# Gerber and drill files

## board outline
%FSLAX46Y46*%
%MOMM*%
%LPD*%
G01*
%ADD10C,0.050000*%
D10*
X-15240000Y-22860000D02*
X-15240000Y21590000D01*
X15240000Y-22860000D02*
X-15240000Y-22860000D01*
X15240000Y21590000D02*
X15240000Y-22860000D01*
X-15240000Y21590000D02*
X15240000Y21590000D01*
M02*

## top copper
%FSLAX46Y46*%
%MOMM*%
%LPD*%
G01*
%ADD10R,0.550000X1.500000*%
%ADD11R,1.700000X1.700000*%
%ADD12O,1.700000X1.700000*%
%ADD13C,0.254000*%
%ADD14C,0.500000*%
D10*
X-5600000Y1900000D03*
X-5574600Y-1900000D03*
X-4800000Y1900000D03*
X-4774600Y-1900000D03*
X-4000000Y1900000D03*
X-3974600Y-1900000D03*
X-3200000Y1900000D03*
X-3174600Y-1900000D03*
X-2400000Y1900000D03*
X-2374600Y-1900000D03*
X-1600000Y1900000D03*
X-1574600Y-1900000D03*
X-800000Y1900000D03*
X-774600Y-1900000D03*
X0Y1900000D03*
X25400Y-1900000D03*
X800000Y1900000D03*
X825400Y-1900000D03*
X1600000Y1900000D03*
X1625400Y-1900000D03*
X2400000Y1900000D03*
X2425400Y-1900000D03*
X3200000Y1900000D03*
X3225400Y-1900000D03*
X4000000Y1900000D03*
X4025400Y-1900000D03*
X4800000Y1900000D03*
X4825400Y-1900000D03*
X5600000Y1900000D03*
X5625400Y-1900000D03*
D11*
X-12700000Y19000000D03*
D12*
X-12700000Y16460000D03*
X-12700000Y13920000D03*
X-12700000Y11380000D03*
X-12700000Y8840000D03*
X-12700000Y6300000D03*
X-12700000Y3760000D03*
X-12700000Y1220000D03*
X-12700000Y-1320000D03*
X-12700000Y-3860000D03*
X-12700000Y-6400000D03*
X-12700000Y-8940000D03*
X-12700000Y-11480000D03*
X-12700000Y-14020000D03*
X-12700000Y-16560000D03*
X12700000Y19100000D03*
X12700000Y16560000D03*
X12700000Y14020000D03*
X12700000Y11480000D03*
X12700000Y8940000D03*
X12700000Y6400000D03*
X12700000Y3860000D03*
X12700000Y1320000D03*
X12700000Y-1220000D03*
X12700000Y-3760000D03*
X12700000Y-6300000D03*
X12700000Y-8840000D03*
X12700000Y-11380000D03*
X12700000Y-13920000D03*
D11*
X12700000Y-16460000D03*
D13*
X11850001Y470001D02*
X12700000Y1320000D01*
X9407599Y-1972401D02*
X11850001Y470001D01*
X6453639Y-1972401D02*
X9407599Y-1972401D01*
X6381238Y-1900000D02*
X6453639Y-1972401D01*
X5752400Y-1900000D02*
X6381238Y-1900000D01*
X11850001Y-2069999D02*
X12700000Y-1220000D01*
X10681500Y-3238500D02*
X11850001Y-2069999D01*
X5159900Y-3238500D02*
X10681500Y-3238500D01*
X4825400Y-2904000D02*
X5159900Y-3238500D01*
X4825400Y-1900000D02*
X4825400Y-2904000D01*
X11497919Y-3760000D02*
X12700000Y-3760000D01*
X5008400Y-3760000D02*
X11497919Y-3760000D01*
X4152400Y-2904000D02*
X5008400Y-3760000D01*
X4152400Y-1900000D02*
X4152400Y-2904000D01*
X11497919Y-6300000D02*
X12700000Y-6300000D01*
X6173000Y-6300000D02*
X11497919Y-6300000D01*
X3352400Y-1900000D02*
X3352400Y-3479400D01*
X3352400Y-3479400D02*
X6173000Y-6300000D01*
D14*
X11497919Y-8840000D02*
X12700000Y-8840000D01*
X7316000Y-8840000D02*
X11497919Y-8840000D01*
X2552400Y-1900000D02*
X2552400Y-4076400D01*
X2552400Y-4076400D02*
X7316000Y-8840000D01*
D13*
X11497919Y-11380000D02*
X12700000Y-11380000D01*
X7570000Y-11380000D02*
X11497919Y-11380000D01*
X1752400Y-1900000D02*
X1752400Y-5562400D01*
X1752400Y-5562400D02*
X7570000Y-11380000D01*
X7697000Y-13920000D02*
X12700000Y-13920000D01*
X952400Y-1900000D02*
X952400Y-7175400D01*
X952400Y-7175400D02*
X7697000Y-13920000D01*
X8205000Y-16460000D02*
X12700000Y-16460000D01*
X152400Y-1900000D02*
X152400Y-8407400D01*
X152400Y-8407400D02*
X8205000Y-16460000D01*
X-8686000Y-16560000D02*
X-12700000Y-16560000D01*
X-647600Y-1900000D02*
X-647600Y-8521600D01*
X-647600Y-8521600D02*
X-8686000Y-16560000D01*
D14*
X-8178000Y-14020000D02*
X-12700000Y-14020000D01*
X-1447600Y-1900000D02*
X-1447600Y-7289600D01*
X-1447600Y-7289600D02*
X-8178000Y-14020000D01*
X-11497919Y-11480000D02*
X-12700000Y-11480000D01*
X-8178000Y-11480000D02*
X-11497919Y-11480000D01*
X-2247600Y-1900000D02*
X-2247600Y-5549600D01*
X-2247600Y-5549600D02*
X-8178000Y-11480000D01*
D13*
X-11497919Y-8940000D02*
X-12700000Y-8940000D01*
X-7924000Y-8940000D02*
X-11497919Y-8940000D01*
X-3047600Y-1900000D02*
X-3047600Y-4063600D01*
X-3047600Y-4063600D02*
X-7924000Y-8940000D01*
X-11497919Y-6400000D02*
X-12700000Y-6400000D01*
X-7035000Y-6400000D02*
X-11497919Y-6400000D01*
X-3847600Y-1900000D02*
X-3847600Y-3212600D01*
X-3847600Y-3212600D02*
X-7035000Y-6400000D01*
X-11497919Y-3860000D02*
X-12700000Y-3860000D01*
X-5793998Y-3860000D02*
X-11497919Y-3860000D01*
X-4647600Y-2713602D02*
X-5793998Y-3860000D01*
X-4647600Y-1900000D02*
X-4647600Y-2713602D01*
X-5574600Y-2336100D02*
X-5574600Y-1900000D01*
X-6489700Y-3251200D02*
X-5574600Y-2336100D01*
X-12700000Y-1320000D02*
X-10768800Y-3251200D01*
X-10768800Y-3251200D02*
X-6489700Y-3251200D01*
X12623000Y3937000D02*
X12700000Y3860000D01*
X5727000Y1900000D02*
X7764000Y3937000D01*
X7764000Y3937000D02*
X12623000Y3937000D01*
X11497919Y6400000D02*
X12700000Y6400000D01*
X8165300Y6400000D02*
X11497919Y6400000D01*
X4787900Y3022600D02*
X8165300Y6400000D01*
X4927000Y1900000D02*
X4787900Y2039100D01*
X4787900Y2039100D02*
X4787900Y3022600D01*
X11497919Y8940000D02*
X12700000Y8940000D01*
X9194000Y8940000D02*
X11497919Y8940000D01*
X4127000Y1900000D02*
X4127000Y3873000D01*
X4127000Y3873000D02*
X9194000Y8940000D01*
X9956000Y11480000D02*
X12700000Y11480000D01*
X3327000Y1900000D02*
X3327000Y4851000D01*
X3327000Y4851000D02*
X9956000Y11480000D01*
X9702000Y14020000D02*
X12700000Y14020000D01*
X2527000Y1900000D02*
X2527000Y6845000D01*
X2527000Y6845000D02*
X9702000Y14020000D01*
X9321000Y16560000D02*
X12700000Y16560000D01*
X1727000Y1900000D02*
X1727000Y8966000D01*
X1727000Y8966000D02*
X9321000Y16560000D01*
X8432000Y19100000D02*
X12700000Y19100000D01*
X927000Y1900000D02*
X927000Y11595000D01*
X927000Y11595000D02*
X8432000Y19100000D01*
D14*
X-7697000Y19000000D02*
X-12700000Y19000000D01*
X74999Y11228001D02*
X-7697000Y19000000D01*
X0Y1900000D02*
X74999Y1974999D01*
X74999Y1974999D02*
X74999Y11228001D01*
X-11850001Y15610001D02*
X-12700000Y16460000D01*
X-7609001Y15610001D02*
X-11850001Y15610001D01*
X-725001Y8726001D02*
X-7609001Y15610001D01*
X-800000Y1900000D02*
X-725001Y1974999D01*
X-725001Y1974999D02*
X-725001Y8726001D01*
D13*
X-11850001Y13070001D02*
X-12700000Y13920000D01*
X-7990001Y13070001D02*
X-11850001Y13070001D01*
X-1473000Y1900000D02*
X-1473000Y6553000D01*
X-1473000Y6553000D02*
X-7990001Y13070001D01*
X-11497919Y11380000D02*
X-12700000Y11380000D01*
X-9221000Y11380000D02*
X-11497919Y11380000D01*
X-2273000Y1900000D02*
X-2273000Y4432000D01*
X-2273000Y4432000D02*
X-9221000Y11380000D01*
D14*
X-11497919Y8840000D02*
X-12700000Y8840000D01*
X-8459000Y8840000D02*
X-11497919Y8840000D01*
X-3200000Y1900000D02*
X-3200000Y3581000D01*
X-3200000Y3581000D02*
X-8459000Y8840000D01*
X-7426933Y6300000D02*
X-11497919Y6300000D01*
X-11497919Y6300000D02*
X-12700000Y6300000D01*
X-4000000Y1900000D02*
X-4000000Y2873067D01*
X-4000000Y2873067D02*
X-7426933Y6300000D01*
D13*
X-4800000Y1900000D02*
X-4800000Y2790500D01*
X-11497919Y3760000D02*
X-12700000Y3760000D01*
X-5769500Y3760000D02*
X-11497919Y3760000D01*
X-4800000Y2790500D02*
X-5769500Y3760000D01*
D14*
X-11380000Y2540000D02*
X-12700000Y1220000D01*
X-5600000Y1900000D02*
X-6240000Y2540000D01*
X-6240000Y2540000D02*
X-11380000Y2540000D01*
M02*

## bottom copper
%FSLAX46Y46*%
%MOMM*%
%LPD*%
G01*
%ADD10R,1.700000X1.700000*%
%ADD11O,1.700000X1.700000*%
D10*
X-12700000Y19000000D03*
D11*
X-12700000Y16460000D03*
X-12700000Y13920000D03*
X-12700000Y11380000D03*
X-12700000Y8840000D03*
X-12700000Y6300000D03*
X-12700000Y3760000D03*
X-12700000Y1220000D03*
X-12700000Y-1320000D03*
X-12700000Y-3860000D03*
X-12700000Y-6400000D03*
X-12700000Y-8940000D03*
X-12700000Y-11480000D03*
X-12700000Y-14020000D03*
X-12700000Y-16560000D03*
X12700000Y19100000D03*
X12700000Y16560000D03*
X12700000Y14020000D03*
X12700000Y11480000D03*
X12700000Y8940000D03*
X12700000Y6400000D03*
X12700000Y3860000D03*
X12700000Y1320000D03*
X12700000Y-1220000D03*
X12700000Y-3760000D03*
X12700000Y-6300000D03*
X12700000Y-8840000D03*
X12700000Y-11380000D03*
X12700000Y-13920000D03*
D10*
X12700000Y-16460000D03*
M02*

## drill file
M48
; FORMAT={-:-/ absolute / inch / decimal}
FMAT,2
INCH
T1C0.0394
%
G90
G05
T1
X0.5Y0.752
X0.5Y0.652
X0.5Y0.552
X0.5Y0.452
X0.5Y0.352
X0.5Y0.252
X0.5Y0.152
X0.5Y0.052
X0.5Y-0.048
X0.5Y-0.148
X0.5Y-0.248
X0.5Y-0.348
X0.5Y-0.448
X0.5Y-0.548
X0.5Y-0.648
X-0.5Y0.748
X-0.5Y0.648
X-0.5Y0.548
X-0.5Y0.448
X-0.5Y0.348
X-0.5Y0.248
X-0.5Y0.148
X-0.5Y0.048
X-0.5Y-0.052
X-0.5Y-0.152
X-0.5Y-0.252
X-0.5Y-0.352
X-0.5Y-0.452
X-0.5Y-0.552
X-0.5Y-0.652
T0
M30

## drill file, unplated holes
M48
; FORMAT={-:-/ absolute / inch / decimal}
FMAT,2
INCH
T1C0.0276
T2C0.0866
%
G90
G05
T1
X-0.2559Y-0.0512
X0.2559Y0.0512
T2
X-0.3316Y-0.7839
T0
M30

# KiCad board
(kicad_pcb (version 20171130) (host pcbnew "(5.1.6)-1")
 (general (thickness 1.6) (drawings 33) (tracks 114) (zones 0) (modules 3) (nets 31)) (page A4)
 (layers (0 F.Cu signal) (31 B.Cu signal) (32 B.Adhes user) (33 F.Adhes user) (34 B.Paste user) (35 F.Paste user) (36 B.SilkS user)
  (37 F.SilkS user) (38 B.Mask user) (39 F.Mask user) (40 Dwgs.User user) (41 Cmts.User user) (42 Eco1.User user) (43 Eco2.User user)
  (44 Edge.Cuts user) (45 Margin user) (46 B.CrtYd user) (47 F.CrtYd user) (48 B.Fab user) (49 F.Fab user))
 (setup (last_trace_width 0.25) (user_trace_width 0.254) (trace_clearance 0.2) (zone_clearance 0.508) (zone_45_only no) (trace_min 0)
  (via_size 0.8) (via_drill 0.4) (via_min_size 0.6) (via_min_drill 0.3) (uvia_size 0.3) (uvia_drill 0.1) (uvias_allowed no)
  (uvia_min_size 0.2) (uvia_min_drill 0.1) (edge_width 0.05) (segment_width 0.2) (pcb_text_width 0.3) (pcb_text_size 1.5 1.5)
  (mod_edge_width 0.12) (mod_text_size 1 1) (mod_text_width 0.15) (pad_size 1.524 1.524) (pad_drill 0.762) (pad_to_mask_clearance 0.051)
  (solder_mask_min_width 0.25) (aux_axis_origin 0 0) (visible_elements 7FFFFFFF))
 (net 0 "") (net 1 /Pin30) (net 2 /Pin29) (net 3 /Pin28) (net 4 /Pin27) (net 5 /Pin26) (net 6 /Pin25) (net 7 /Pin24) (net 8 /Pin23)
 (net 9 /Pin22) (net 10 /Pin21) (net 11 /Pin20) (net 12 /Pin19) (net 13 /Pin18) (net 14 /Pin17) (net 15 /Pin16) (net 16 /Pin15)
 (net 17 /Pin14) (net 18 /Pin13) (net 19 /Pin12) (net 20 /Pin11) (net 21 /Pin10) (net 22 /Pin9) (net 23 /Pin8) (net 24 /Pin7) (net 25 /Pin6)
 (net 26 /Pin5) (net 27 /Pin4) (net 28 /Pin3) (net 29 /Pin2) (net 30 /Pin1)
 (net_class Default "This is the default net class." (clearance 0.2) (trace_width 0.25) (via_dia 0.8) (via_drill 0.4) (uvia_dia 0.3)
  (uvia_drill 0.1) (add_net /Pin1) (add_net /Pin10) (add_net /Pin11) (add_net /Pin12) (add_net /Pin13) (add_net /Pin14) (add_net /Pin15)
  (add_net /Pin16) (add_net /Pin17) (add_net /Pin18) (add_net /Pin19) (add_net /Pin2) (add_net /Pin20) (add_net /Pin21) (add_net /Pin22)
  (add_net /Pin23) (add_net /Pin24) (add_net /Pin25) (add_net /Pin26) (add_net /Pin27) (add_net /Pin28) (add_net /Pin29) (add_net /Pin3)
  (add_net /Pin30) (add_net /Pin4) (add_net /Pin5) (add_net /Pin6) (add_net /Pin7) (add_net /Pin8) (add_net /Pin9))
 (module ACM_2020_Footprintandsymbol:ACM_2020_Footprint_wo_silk (layer F.Cu) (at 0 0)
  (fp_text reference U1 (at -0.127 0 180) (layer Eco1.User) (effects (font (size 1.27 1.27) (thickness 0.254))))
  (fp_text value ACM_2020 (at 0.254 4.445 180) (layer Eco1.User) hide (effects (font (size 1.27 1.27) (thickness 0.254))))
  (pad 30 smd rect (at -5.6 -1.9) (size 0.55 1.5) (layers F.Cu F.Paste F.Mask) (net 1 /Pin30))
  (pad 29 smd rect (at -5.5746 1.9) (size 0.55 1.5) (layers F.Cu F.Paste F.Mask) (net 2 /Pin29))
  (pad 28 smd rect (at -4.8 -1.9) (size 0.55 1.5) (layers F.Cu F.Paste F.Mask) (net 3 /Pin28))
  (pad 27 smd rect (at -4.7746 1.9) (size 0.55 1.5) (layers F.Cu F.Paste F.Mask) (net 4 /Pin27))
  (pad 26 smd rect (at -4 -1.9) (size 0.55 1.5) (layers F.Cu F.Paste F.Mask) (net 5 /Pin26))
  (pad 25 smd rect (at -3.9746 1.9) (size 0.55 1.5) (layers F.Cu F.Paste F.Mask) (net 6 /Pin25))
  (pad 24 smd rect (at -3.2 -1.9) (size 0.55 1.5) (layers F.Cu F.Paste F.Mask) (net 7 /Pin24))
  (pad 23 smd rect (at -3.1746 1.9) (size 0.55 1.5) (layers F.Cu F.Paste F.Mask) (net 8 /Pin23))
  (pad 22 smd rect (at -2.4 -1.9) (size 0.55 1.5) (layers F.Cu F.Paste F.Mask) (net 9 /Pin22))
  (pad 21 smd rect (at -2.3746 1.9) (size 0.55 1.5) (layers F.Cu F.Paste F.Mask) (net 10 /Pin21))
  (pad 20 smd rect (at -1.6 -1.9) (size 0.55 1.5) (layers F.Cu F.Paste F.Mask) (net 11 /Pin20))
  (pad 19 smd rect (at -1.5746 1.9) (size 0.55 1.5) (layers F.Cu F.Paste F.Mask) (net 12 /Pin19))
  (pad 18 smd rect (at -0.8 -1.9) (size 0.55 1.5) (layers F.Cu F.Paste F.Mask) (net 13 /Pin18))
  (pad 17 smd rect (at -0.7746 1.9) (size 0.55 1.5) (layers F.Cu F.Paste F.Mask) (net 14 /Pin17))
  (pad 16 smd rect (at 0 -1.9) (size 0.55 1.5) (layers F.Cu F.Paste F.Mask) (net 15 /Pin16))
  (pad 15 smd rect (at 0.0254 1.9) (size 0.55 1.5) (layers F.Cu F.Paste F.Mask) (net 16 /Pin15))
  (pad 14 smd rect (at 0.8 -1.9) (size 0.55 1.5) (layers F.Cu F.Paste F.Mask) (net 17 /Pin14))
  (pad 13 smd rect (at 0.8254 1.9) (size 0.55 1.5) (layers F.Cu F.Paste F.Mask) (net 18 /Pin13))
  (pad 12 smd rect (at 1.6 -1.9) (size 0.55 1.5) (layers F.Cu F.Paste F.Mask) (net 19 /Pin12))
  (pad 11 smd rect (at 1.6254 1.9) (size 0.55 1.5) (layers F.Cu F.Paste F.Mask) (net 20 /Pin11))
  (pad 10 smd rect (at 2.4 -1.9) (size 0.55 1.5) (layers F.Cu F.Paste F.Mask) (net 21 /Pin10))
  (pad 9 smd rect (at 2.4254 1.9) (size 0.55 1.5) (layers F.Cu F.Paste F.Mask) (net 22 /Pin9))
  (pad 8 smd rect (at 3.2 -1.9) (size 0.55 1.5) (layers F.Cu F.Paste F.Mask) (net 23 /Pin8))
  (pad 7 smd rect (at 3.2254 1.9) (size 0.55 1.5) (layers F.Cu F.Paste F.Mask) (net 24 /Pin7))
  (pad 6 smd rect (at 4 -1.9) (size 0.55 1.5) (layers F.Cu F.Paste F.Mask) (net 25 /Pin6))
  (pad 5 smd rect (at 4.0254 1.9) (size 0.55 1.5) (layers F.Cu F.Paste F.Mask) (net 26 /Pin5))
  (pad 4 smd rect (at 4.8 -1.9) (size 0.55 1.5) (layers F.Cu F.Paste F.Mask) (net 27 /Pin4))
  (pad 3 smd rect (at 4.8254 1.9) (size 0.55 1.5) (layers F.Cu F.Paste F.Mask) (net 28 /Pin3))
  (pad 2 smd rect (at 5.6 -1.9) (size 0.55 1.5) (layers F.Cu F.Paste F.Mask) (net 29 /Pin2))
  (pad 1 smd rect (at 5.6254 1.9) (size 0.55 1.5) (layers F.Cu F.Paste F.Mask) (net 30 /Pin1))
  (pad "" np_thru_hole circle (at -6.5 1.3) (size 0.7 0.7) (drill 0.7) (layers *.Cu *.Mask))
  (pad "" np_thru_hole circle (at 6.5 -1.3) (size 0.7 0.7) (drill 0.7) (layers *.Cu *.Mask))
  (pad "" np_thru_hole circle (at -8.422 19.912) (size 2.2 2.2) (drill 2.2) (layers *.Cu *.Mask)))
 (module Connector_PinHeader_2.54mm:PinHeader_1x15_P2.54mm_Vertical (layer F.Cu) (at -12.7 -19)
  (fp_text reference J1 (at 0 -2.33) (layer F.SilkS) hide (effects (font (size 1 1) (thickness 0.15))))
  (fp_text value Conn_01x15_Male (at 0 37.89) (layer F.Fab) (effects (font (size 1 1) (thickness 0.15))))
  (pad 1 thru_hole rect (at 0 0) (size 1.7 1.7) (drill 1) (layers *.Cu *.Mask) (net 15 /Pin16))
  (pad 2 thru_hole oval (at 0 2.54) (size 1.7 1.7) (drill 1) (layers *.Cu *.Mask) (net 13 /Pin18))
  (pad 3 thru_hole oval (at 0 5.08) (size 1.7 1.7) (drill 1) (layers *.Cu *.Mask) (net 11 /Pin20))
  (pad 4 thru_hole oval (at 0 7.62) (size 1.7 1.7) (drill 1) (layers *.Cu *.Mask) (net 9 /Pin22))
  (pad 5 thru_hole oval (at 0 10.16) (size 1.7 1.7) (drill 1) (layers *.Cu *.Mask) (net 7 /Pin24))
  (pad 6 thru_hole oval (at 0 12.7) (size 1.7 1.7) (drill 1) (layers *.Cu *.Mask) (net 5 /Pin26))
  (pad 7 thru_hole oval (at 0 15.24) (size 1.7 1.7) (drill 1) (layers *.Cu *.Mask) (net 3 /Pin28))
  (pad 8 thru_hole oval (at 0 17.78) (size 1.7 1.7) (drill 1) (layers *.Cu *.Mask) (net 1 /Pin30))
  (pad 9 thru_hole oval (at 0 20.32) (size 1.7 1.7) (drill 1) (layers *.Cu *.Mask) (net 2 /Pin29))
  (pad 10 thru_hole oval (at 0 22.86) (size 1.7 1.7) (drill 1) (layers *.Cu *.Mask) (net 4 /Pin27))
  (pad 11 thru_hole oval (at 0 25.4) (size 1.7 1.7) (drill 1) (layers *.Cu *.Mask) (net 6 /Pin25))
  (pad 12 thru_hole oval (at 0 27.94) (size 1.7 1.7) (drill 1) (layers *.Cu *.Mask) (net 8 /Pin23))
  (pad 13 thru_hole oval (at 0 30.48) (size 1.7 1.7) (drill 1) (layers *.Cu *.Mask) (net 10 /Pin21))
  (pad 14 thru_hole oval (at 0 33.02) (size 1.7 1.7) (drill 1) (layers *.Cu *.Mask) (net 12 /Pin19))
  (pad 15 thru_hole oval (at 0 35.56) (size 1.7 1.7) (drill 1) (layers *.Cu *.Mask) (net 14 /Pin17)))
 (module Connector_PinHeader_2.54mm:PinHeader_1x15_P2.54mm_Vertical (layer F.Cu) (at 12.7 16.46 180)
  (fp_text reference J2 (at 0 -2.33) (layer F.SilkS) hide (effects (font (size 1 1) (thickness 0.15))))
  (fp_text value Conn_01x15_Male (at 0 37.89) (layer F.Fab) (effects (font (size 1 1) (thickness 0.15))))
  (pad 15 thru_hole oval (at 0 35.56 180) (size 1.7 1.7) (drill 1) (layers *.Cu *.Mask) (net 17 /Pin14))
  (pad 14 thru_hole oval (at 0 33.02 180) (size 1.7 1.7) (drill 1) (layers *.Cu *.Mask) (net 19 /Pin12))
  (pad 13 thru_hole oval (at 0 30.48 180) (size 1.7 1.7) (drill 1) (layers *.Cu *.Mask) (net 21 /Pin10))
  (pad 12 thru_hole oval (at 0 27.94 180) (size 1.7 1.7) (drill 1) (layers *.Cu *.Mask) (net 23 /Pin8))
  (pad 11 thru_hole oval (at 0 25.4 180) (size 1.7 1.7) (drill 1) (layers *.Cu *.Mask) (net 25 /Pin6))
  (pad 10 thru_hole oval (at 0 22.86 180) (size 1.7 1.7) (drill 1) (layers *.Cu *.Mask) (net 27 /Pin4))
  (pad 9 thru_hole oval (at 0 20.32 180) (size 1.7 1.7) (drill 1) (layers *.Cu *.Mask) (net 29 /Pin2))
  (pad 8 thru_hole oval (at 0 17.78 180) (size 1.7 1.7) (drill 1) (layers *.Cu *.Mask) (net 30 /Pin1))
  (pad 7 thru_hole oval (at 0 15.24 180) (size 1.7 1.7) (drill 1) (layers *.Cu *.Mask) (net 28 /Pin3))
  (pad 6 thru_hole oval (at 0 12.7 180) (size 1.7 1.7) (drill 1) (layers *.Cu *.Mask) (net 26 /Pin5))
  (pad 5 thru_hole oval (at 0 10.16 180) (size 1.7 1.7) (drill 1) (layers *.Cu *.Mask) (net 24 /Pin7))
  (pad 4 thru_hole oval (at 0 7.62 180) (size 1.7 1.7) (drill 1) (layers *.Cu *.Mask) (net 22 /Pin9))
  (pad 3 thru_hole oval (at 0 5.08 180) (size 1.7 1.7) (drill 1) (layers *.Cu *.Mask) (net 20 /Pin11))
  (pad 2 thru_hole oval (at 0 2.54 180) (size 1.7 1.7) (drill 1) (layers *.Cu *.Mask) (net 18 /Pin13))
  (pad 1 thru_hole rect (at 0 0 180) (size 1.7 1.7) (drill 1) (layers *.Cu *.Mask) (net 16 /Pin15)))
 (gr_line (start -15.24 22.86) (end -15.24 -21.59) (layer Edge.Cuts) (width 0.05))
 (gr_line (start 15.24 22.86) (end -15.24 22.86) (layer Edge.Cuts) (width 0.05))
 (gr_line (start 15.24 -21.59) (end 15.24 22.86) (layer Edge.Cuts) (width 0.05))
 (gr_line (start -15.24 -21.59) (end 15.24 -21.59) (layer Edge.Cuts) (width 0.05))
 (segment (start 11.850001 -0.470001) (end 12.7 -1.32) (width 0.254) (layer F.Cu) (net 30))
 (segment (start 9.407599 1.972401) (end 11.850001 -0.470001) (width 0.254) (layer F.Cu) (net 30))
 (segment (start 6.453639 1.972401) (end 9.407599 1.972401) (width 0.254) (layer F.Cu) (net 30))
 (segment (start 6.381238 1.9) (end 6.453639 1.972401) (width 0.254) (layer F.Cu) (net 30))
 (segment (start 5.7524 1.9) (end 6.381238 1.9) (width 0.254) (layer F.Cu) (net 30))
 (segment (start 11.850001 2.069999) (end 12.7 1.22) (width 0.254) (layer F.Cu) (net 28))
 (segment (start 10.6815 3.2385) (end 11.850001 2.069999) (width 0.254) (layer F.Cu) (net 28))
 (segment (start 5.1599 3.2385) (end 10.6815 3.2385) (width 0.254) (layer F.Cu) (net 28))
 (segment (start 4.8254 2.904) (end 5.1599 3.2385) (width 0.254) (layer F.Cu) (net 28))
 (segment (start 4.8254 1.9) (end 4.8254 2.904) (width 0.254) (layer F.Cu) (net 28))
 (segment (start 11.497919 3.76) (end 12.7 3.76) (width 0.254) (layer F.Cu) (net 26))
 (segment (start 5.0084 3.76) (end 11.497919 3.76) (width 0.254) (layer F.Cu) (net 26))
 (segment (start 4.1524 2.904) (end 5.0084 3.76) (width 0.254) (layer F.Cu) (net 26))
 (segment (start 4.1524 1.9) (end 4.1524 2.904) (width 0.254) (layer F.Cu) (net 26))
 (segment (start 11.497919 6.3) (end 12.7 6.3) (width 0.254) (layer F.Cu) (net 24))
 (segment (start 6.173 6.3) (end 11.497919 6.3) (width 0.254) (layer F.Cu) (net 24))
 (segment (start 3.3524 1.9) (end 3.3524 3.4794) (width 0.254) (layer F.Cu) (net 24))
 (segment (start 3.3524 3.4794) (end 6.173 6.3) (width 0.254) (layer F.Cu) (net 24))
 (segment (start 11.497919 8.84) (end 12.7 8.84) (width 0.5) (layer F.Cu) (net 22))
 (segment (start 7.316 8.84) (end 11.497919 8.84) (width 0.5) (layer F.Cu) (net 22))
 (segment (start 2.5524 1.9) (end 2.5524 4.0764) (width 0.5) (layer F.Cu) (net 22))
 (segment (start 2.5524 4.0764) (end 7.316 8.84) (width 0.5) (layer F.Cu) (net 22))
 (segment (start 11.497919 11.38) (end 12.7 11.38) (width 0.254) (layer F.Cu) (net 20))
 (segment (start 7.57 11.38) (end 11.497919 11.38) (width 0.254) (layer F.Cu) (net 20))
 (segment (start 1.7524 1.9) (end 1.7524 5.5624) (width 0.254) (layer F.Cu) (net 20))
 (segment (start 1.7524 5.5624) (end 7.57 11.38) (width 0.254) (layer F.Cu) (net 20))
 (segment (start 7.697 13.92) (end 12.7 13.92) (width 0.254) (layer F.Cu) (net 18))
 (segment (start 0.9524 1.9) (end 0.9524 7.1754) (width 0.254) (layer F.Cu) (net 18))
 (segment (start 0.9524 7.1754) (end 7.697 13.92) (width 0.254) (layer F.Cu) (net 18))
 (segment (start 8.205 16.46) (end 12.7 16.46) (width 0.254) (layer F.Cu) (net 16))
 (segment (start 0.1524 1.9) (end 0.1524 8.4074) (width 0.254) (layer F.Cu) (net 16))
 (segment (start 0.1524 8.4074) (end 8.205 16.46) (width 0.254) (layer F.Cu) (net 16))
 (segment (start -8.686 16.56) (end -12.7 16.56) (width 0.254) (layer F.Cu) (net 14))
 (segment (start -0.6476 1.9) (end -0.6476 8.5216) (width 0.254) (layer F.Cu) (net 14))
 (segment (start -0.6476 8.5216) (end -8.686 16.56) (width 0.254) (layer F.Cu) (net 14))
 (segment (start -8.178 14.02) (end -12.7 14.02) (width 0.5) (layer F.Cu) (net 12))
 (segment (start -1.4476 1.9) (end -1.4476 7.2896) (width 0.5) (layer F.Cu) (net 12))
 (segment (start -1.4476 7.2896) (end -8.178 14.02) (width 0.5) (layer F.Cu) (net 12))
 (segment (start -11.497919 11.48) (end -12.7 11.48) (width 0.5) (layer F.Cu) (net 10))
 (segment (start -8.178 11.48) (end -11.497919 11.48) (width 0.5) (layer F.Cu) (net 10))
 (segment (start -2.2476 1.9) (end -2.2476 5.5496) (width 0.5) (layer F.Cu) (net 10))
 (segment (start -2.2476 5.5496) (end -8.178 11.48) (width 0.5) (layer F.Cu) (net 10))
 (segment (start -11.497919 8.94) (end -12.7 8.94) (width 0.254) (layer F.Cu) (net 8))
 (segment (start -7.924 8.94) (end -11.497919 8.94) (width 0.254) (layer F.Cu) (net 8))
 (segment (start -3.0476 1.9) (end -3.0476 4.0636) (width 0.254) (layer F.Cu) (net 8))
 (segment (start -3.0476 4.0636) (end -7.924 8.94) (width 0.254) (layer F.Cu) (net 8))
 (segment (start -11.497919 6.4) (end -12.7 6.4) (width 0.254) (layer F.Cu) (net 6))
 (segment (start -7.035 6.4) (end -11.497919 6.4) (width 0.254) (layer F.Cu) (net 6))
 (segment (start -3.8476 1.9) (end -3.8476 3.2126) (width 0.254) (layer F.Cu) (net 6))
 (segment (start -3.8476 3.2126) (end -7.035 6.4) (width 0.254) (layer F.Cu) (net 6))
 (segment (start -11.497919 3.86) (end -12.7 3.86) (width 0.254) (layer F.Cu) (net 4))
 (segment (start -5.793998 3.86) (end -11.497919 3.86) (width 0.254) (layer F.Cu) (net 4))
 (segment (start -4.6476 2.713602) (end -5.793998 3.86) (width 0.254) (layer F.Cu) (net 4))
 (segment (start -4.6476 1.9) (end -4.6476 2.713602) (width 0.254) (layer F.Cu) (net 4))
 (segment (start -5.5746 2.3361) (end -5.5746 1.9) (width 0.254) (layer F.Cu) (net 2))
 (segment (start -6.4897 3.2512) (end -5.5746 2.3361) (width 0.254) (layer F.Cu) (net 2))
 (segment (start -12.7 1.32) (end -10.7688 3.2512) (width 0.254) (layer F.Cu) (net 2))
 (segment (start -10.7688 3.2512) (end -6.4897 3.2512) (width 0.254) (layer F.Cu) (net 2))
 (segment (start 12.623 -3.937) (end 12.7 -3.86) (width 0.254) (layer F.Cu) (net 29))
 (segment (start 5.727 -1.9) (end 7.764 -3.937) (width 0.254) (layer F.Cu) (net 29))
 (segment (start 7.764 -3.937) (end 12.623 -3.937) (width 0.254) (layer F.Cu) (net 29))
 (segment (start 11.497919 -6.4) (end 12.7 -6.4) (width 0.254) (layer F.Cu) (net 27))
 (segment (start 8.1653 -6.4) (end 11.497919 -6.4) (width 0.254) (layer F.Cu) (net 27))
 (segment (start 4.7879 -3.0226) (end 8.1653 -6.4) (width 0.254) (layer F.Cu) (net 27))
 (segment (start 4.927 -1.9) (end 4.7879 -2.0391) (width 0.254) (layer F.Cu) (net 27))
 (segment (start 4.7879 -2.0391) (end 4.7879 -3.0226) (width 0.254) (layer F.Cu) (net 27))
 (segment (start 11.497919 -8.94) (end 12.7 -8.94) (width 0.254) (layer F.Cu) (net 25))
 (segment (start 9.194 -8.94) (end 11.497919 -8.94) (width 0.254) (layer F.Cu) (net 25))
 (segment (start 4.127 -1.9) (end 4.127 -3.873) (width 0.254) (layer F.Cu) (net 25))
 (segment (start 4.127 -3.873) (end 9.194 -8.94) (width 0.254) (layer F.Cu) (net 25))
 (segment (start 9.956 -11.48) (end 12.7 -11.48) (width 0.254) (layer F.Cu) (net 23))
 (segment (start 3.327 -1.9) (end 3.327 -4.851) (width 0.254) (layer F.Cu) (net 23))
 (segment (start 3.327 -4.851) (end 9.956 -11.48) (width 0.254) (layer F.Cu) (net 23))
 (segment (start 9.702 -14.02) (end 12.7 -14.02) (width 0.254) (layer F.Cu) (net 21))
 (segment (start 2.527 -1.9) (end 2.527 -6.845) (width 0.254) (layer F.Cu) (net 21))
 (segment (start 2.527 -6.845) (end 9.702 -14.02) (width 0.254) (layer F.Cu) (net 21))
 (segment (start 9.321 -16.56) (end 12.7 -16.56) (width 0.254) (layer F.Cu) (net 19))
 (segment (start 1.727 -1.9) (end 1.727 -8.966) (width 0.254) (layer F.Cu) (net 19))
 (segment (start 1.727 -8.966) (end 9.321 -16.56) (width 0.254) (layer F.Cu) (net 19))
 (segment (start 8.432 -19.1) (end 12.7 -19.1) (width 0.254) (layer F.Cu) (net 17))
 (segment (start 0.927 -1.9) (end 0.927 -11.595) (width 0.254) (layer F.Cu) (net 17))
 (segment (start 0.927 -11.595) (end 8.432 -19.1) (width 0.254) (layer F.Cu) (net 17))
 (segment (start -7.697 -19) (end -12.7 -19) (width 0.5) (layer F.Cu) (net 15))
 (segment (start 0.074999 -11.228001) (end -7.697 -19) (width 0.5) (layer F.Cu) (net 15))
 (segment (start 0 -1.9) (end 0.074999 -1.974999) (width 0.5) (layer F.Cu) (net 15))
 (segment (start 0.074999 -1.974999) (end 0.074999 -11.228001) (width 0.5) (layer F.Cu) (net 15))
 (segment (start -11.850001 -15.610001) (end -12.7 -16.46) (width 0.5) (layer F.Cu) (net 13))
 (segment (start -7.609001 -15.610001) (end -11.850001 -15.610001) (width 0.5) (layer F.Cu) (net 13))
 (segment (start -0.725001 -8.726001) (end -7.609001 -15.610001) (width 0.5) (layer F.Cu) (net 13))
 (segment (start -0.8 -1.9) (end -0.725001 -1.974999) (width 0.5) (layer F.Cu) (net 13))
 (segment (start -0.725001 -1.974999) (end -0.725001 -8.726001) (width 0.5) (layer F.Cu) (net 13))
 (segment (start -11.850001 -13.070001) (end -12.7 -13.92) (width 0.254) (layer F.Cu) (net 11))
 (segment (start -7.990001 -13.070001) (end -11.850001 -13.070001) (width 0.254) (layer F.Cu) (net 11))
 (segment (start -1.473 -1.9) (end -1.473 -6.553) (width 0.254) (layer F.Cu) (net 11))
 (segment (start -1.473 -6.553) (end -7.990001 -13.070001) (width 0.254) (layer F.Cu) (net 11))
 (segment (start -11.497919 -11.38) (end -12.7 -11.38) (width 0.254) (layer F.Cu) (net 9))
 (segment (start -9.221 -11.38) (end -11.497919 -11.38) (width 0.254) (layer F.Cu) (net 9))
 (segment (start -2.273 -1.9) (end -2.273 -4.432) (width 0.254) (layer F.Cu) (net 9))
 (segment (start -2.273 -4.432) (end -9.221 -11.38) (width 0.254) (layer F.Cu) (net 9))
 (segment (start -11.497919 -8.84) (end -12.7 -8.84) (width 0.5) (layer F.Cu) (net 7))
 (segment (start -8.459 -8.84) (end -11.497919 -8.84) (width 0.5) (layer F.Cu) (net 7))
 (segment (start -3.2 -1.9) (end -3.2 -3.581) (width 0.5) (layer F.Cu) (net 7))
 (segment (start -3.2 -3.581) (end -8.459 -8.84) (width 0.5) (layer F.Cu) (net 7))
 (segment (start -7.426933 -6.3) (end -11.497919 -6.3) (width 0.5) (layer F.Cu) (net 5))
 (segment (start -11.497919 -6.3) (end -12.7 -6.3) (width 0.5) (layer F.Cu) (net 5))
 (segment (start -4 -1.9) (end -4 -2.873067) (width 0.5) (layer F.Cu) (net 5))
 (segment (start -4 -2.873067) (end -7.426933 -6.3) (width 0.5) (layer F.Cu) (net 5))
 (segment (start -4.8 -1.9) (end -4.8 -2.7905) (width 0.254) (layer F.Cu) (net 3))
 (segment (start -11.497919 -3.76) (end -12.7 -3.76) (width 0.254) (layer F.Cu) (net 3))
 (segment (start -5.7695 -3.76) (end -11.497919 -3.76) (width 0.254) (layer F.Cu) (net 3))
 (segment (start -4.8 -2.7905) (end -5.7695 -3.76) (width 0.254) (layer F.Cu) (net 3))
 (segment (start -11.38 -2.54) (end -12.7 -1.22) (width 0.5) (layer F.Cu) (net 1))
 (segment (start -5.6 -1.9) (end -6.24 -2.54) (width 0.5) (layer F.Cu) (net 1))
 (segment (start -6.24 -2.54) (end -11.38 -2.54) (width 0.5) (layer F.Cu) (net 1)))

